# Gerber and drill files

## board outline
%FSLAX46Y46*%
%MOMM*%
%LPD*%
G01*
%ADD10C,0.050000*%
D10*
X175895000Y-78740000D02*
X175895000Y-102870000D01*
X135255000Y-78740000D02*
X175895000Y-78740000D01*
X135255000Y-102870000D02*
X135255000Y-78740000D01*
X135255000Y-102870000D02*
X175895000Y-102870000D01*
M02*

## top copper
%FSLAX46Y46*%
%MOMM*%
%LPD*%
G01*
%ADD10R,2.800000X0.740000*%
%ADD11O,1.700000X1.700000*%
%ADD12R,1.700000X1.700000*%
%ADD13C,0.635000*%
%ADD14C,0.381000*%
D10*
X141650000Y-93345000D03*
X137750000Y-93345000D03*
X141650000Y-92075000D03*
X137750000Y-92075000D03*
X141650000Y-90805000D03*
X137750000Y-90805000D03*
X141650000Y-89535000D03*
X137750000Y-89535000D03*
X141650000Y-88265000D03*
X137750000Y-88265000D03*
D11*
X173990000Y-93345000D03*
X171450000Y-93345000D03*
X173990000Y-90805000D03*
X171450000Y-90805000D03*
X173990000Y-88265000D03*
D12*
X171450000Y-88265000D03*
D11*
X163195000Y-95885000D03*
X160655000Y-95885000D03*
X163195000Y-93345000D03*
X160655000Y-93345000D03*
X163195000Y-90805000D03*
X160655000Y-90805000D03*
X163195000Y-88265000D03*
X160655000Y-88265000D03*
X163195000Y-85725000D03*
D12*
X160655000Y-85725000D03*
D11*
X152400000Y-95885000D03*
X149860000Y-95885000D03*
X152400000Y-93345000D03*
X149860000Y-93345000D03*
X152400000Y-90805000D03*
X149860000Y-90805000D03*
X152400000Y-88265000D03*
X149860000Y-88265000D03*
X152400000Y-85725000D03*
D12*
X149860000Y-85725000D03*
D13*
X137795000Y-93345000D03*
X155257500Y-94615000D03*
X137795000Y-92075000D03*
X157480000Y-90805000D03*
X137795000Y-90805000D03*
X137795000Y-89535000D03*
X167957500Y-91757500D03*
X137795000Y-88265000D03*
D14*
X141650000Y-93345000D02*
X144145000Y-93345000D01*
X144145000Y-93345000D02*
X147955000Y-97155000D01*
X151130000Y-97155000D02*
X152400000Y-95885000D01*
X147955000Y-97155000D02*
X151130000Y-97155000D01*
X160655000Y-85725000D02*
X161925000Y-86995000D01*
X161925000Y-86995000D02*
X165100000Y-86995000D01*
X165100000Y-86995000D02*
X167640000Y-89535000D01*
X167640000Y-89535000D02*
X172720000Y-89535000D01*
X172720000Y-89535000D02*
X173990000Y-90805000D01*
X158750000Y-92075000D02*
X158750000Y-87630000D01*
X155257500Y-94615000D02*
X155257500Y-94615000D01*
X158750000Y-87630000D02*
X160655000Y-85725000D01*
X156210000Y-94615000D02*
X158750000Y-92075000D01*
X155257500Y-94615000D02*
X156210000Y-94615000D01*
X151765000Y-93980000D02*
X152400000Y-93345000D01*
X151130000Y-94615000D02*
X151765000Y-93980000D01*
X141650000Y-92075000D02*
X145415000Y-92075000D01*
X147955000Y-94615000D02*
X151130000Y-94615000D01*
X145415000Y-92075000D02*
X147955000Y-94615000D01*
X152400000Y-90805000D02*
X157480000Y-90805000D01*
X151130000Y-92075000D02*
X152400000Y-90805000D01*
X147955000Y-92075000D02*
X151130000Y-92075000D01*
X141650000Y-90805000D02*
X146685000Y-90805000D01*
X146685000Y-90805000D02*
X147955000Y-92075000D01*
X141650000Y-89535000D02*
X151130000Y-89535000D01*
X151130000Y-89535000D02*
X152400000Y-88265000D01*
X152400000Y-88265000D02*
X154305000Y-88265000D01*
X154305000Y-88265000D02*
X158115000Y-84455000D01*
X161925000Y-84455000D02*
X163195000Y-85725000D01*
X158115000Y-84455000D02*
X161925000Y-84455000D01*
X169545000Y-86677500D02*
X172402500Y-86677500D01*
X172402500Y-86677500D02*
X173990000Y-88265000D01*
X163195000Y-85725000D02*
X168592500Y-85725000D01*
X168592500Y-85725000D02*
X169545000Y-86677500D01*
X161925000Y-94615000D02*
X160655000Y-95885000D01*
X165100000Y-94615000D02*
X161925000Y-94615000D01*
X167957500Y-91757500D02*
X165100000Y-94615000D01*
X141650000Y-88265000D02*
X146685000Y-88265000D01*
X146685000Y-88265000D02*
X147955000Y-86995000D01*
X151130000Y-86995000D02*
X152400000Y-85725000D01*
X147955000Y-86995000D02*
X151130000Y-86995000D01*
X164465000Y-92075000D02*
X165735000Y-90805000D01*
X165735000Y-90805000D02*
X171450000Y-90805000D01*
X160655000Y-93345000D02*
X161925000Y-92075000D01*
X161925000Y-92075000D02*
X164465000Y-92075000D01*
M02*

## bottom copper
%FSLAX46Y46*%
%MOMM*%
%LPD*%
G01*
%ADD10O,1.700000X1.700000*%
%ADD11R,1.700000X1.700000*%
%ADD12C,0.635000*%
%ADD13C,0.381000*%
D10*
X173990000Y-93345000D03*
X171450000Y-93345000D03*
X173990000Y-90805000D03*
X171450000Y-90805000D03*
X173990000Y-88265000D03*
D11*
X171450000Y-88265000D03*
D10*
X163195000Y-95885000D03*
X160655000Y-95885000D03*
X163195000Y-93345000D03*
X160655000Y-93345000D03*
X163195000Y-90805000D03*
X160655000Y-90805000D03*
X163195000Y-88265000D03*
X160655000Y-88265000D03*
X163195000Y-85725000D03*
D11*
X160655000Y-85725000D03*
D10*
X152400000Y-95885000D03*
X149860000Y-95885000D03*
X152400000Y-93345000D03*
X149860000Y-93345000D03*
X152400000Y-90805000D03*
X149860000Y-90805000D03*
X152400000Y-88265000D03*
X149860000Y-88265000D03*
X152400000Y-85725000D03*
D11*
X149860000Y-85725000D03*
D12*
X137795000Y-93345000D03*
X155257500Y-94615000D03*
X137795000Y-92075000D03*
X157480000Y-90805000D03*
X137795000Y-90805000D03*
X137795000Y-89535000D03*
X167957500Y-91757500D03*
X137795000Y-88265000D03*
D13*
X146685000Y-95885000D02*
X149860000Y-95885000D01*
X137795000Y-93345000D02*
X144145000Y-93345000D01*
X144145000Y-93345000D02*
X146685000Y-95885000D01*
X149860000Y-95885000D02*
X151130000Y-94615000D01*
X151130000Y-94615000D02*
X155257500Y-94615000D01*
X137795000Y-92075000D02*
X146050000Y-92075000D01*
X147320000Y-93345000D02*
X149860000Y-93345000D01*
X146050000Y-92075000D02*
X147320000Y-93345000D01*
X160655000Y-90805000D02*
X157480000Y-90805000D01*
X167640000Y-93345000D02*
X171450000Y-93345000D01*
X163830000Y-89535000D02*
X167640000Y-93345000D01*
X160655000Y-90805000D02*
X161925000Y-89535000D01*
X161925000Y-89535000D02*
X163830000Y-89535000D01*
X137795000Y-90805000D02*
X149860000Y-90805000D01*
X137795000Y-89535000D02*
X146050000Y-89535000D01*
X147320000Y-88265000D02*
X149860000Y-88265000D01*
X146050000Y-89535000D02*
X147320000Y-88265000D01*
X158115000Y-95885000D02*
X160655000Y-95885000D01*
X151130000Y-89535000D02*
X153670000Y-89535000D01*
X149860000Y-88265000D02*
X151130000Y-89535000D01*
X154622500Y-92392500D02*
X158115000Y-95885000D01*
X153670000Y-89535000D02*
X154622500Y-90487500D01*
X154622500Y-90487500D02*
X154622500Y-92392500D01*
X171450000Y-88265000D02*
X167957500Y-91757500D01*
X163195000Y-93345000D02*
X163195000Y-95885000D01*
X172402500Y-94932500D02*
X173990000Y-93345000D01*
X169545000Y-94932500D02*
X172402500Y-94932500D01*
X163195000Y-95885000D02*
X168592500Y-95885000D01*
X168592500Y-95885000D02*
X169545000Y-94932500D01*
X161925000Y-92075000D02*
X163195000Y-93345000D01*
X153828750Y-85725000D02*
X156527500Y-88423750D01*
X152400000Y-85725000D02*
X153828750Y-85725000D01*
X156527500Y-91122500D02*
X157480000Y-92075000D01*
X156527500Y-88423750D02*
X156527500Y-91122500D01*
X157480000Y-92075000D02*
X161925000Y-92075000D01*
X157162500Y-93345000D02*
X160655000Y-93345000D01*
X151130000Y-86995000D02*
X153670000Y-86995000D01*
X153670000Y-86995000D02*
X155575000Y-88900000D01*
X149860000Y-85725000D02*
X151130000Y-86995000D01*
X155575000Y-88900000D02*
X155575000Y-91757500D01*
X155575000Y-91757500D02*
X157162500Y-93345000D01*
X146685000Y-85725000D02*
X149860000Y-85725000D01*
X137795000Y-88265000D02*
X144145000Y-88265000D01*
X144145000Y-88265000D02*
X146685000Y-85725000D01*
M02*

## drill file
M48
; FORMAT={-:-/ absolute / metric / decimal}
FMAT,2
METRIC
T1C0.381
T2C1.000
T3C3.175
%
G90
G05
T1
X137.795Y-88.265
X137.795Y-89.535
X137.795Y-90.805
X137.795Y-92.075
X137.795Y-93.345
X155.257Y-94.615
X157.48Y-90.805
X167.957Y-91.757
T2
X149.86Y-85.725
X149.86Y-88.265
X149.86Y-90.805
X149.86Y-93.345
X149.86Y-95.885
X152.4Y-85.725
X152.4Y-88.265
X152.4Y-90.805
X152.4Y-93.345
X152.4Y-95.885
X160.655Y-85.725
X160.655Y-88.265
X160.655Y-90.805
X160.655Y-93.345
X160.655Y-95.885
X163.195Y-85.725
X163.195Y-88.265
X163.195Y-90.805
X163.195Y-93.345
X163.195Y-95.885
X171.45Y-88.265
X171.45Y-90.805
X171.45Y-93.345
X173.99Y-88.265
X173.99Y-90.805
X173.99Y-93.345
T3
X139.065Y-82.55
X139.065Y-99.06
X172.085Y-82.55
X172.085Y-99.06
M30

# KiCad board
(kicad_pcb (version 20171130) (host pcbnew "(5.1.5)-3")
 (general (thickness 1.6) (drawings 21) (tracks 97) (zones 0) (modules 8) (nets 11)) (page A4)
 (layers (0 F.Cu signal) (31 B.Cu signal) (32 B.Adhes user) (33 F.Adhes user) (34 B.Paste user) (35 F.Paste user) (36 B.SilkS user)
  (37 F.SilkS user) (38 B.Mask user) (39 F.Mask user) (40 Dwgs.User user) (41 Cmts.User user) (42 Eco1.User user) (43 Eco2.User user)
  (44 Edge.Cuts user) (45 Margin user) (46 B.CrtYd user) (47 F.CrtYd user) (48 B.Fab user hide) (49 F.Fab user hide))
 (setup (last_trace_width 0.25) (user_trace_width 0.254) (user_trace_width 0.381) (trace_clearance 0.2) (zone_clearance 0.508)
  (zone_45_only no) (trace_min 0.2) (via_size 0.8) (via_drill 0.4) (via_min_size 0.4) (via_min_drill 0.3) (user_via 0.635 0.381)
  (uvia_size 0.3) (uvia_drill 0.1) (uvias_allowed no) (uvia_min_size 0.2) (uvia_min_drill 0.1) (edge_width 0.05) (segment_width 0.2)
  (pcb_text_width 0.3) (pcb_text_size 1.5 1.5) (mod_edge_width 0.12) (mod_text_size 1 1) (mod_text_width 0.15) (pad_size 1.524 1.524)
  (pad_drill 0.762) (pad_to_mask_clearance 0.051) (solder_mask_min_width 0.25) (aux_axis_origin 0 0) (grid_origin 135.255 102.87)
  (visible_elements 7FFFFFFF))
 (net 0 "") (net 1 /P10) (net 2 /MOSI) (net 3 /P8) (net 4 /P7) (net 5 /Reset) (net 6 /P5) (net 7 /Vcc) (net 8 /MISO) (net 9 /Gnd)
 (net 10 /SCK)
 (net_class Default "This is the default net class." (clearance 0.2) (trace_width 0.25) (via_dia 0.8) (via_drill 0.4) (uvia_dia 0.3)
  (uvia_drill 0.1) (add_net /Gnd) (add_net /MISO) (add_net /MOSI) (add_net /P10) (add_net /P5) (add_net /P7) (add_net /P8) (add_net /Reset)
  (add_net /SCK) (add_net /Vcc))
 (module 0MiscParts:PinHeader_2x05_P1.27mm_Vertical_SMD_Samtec (layer F.Cu) (at 139.7 90.805)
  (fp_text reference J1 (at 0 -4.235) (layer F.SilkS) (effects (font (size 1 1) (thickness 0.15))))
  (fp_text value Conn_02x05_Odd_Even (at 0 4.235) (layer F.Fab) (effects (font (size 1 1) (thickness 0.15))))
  (pad 10 smd rect (at 1.95 2.54) (size 2.8 0.74) (layers F.Cu F.Paste F.Mask) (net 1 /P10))
  (pad 9 smd rect (at -1.95 2.54) (size 2.8 0.74) (layers F.Cu F.Paste F.Mask) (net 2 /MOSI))
  (pad 8 smd rect (at 1.95 1.27) (size 2.8 0.74) (layers F.Cu F.Paste F.Mask) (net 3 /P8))
  (pad 7 smd rect (at -1.95 1.27) (size 2.8 0.74) (layers F.Cu F.Paste F.Mask) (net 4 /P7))
  (pad 6 smd rect (at 1.95 0) (size 2.8 0.74) (layers F.Cu F.Paste F.Mask) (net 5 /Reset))
  (pad 5 smd rect (at -1.95 0) (size 2.8 0.74) (layers F.Cu F.Paste F.Mask) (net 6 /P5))
  (pad 4 smd rect (at 1.95 -1.27) (size 2.8 0.74) (layers F.Cu F.Paste F.Mask) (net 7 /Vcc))
  (pad 3 smd rect (at -1.95 -1.27) (size 2.8 0.74) (layers F.Cu F.Paste F.Mask) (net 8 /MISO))
  (pad 2 smd rect (at 1.95 -2.54) (size 2.8 0.74) (layers F.Cu F.Paste F.Mask) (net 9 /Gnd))
  (pad 1 smd rect (at -1.95 -2.54) (size 2.8 0.74) (layers F.Cu F.Paste F.Mask) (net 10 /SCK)))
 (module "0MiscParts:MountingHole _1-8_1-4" (layer F.Cu) (at 172.085 82.55)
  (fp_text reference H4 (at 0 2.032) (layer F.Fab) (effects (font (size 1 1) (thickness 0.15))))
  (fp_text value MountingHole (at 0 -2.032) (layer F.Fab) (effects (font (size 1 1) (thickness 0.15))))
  (pad "" np_thru_hole circle (at 0 0) (size 3.175 3.175) (drill 3.175) (layers *.Cu *.Mask)))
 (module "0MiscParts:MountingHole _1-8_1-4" (layer F.Cu) (at 172.085 99.06)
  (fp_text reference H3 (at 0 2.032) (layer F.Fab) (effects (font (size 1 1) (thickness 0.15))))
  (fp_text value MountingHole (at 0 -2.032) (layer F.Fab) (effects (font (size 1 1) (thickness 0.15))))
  (pad "" np_thru_hole circle (at 0 0) (size 3.175 3.175) (drill 3.175) (layers *.Cu *.Mask)))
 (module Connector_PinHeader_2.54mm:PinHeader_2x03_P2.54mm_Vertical (layer F.Cu) (at 171.45 88.265)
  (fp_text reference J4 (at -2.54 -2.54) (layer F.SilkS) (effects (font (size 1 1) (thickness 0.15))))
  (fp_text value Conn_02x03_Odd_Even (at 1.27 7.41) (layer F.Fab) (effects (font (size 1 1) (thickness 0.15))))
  (pad 6 thru_hole oval (at 2.54 5.08) (size 1.7 1.7) (drill 1) (layers *.Cu *.Mask) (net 9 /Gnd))
  (pad 5 thru_hole oval (at 0 5.08) (size 1.7 1.7) (drill 1) (layers *.Cu *.Mask) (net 5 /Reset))
  (pad 4 thru_hole oval (at 2.54 2.54) (size 1.7 1.7) (drill 1) (layers *.Cu *.Mask) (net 2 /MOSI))
  (pad 3 thru_hole oval (at 0 2.54) (size 1.7 1.7) (drill 1) (layers *.Cu *.Mask) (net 10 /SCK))
  (pad 2 thru_hole oval (at 2.54 0) (size 1.7 1.7) (drill 1) (layers *.Cu *.Mask) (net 7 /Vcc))
  (pad 1 thru_hole rect (at 0 0) (size 1.7 1.7) (drill 1) (layers *.Cu *.Mask) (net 8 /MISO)))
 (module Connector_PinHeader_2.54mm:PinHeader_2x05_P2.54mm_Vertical (layer F.Cu) (at 160.655 85.725)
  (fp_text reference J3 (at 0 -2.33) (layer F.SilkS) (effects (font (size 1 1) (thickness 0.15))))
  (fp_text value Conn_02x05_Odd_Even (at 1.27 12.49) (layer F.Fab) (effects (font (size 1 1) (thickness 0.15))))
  (pad 10 thru_hole oval (at 2.54 10.16) (size 1.7 1.7) (drill 1) (layers *.Cu *.Mask) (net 9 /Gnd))
  (pad 9 thru_hole oval (at 0 10.16) (size 1.7 1.7) (drill 1) (layers *.Cu *.Mask) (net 8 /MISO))
  (pad 8 thru_hole oval (at 2.54 7.62) (size 1.7 1.7) (drill 1) (layers *.Cu *.Mask) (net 9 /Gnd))
  (pad 7 thru_hole oval (at 0 7.62) (size 1.7 1.7) (drill 1) (layers *.Cu *.Mask) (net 10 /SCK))
  (pad 6 thru_hole oval (at 2.54 5.08) (size 1.7 1.7) (drill 1) (layers *.Cu *.Mask))
  (pad 5 thru_hole oval (at 0 5.08) (size 1.7 1.7) (drill 1) (layers *.Cu *.Mask) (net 5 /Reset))
  (pad 4 thru_hole oval (at 2.54 2.54) (size 1.7 1.7) (drill 1) (layers *.Cu *.Mask))
  (pad 3 thru_hole oval (at 0 2.54) (size 1.7 1.7) (drill 1) (layers *.Cu *.Mask))
  (pad 2 thru_hole oval (at 2.54 0) (size 1.7 1.7) (drill 1) (layers *.Cu *.Mask) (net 7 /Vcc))
  (pad 1 thru_hole rect (at 0 0) (size 1.7 1.7) (drill 1) (layers *.Cu *.Mask) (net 2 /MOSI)))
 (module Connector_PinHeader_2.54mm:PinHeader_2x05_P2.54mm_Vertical (layer F.Cu) (at 149.86 85.725)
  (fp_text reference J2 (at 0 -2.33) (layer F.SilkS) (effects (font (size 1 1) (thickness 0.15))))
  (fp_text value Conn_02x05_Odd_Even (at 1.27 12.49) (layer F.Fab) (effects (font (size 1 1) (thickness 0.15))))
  (pad 10 thru_hole oval (at 2.54 10.16) (size 1.7 1.7) (drill 1) (layers *.Cu *.Mask) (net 1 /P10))
  (pad 9 thru_hole oval (at 0 10.16) (size 1.7 1.7) (drill 1) (layers *.Cu *.Mask) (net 2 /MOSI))
  (pad 8 thru_hole oval (at 2.54 7.62) (size 1.7 1.7) (drill 1) (layers *.Cu *.Mask) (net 3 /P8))
  (pad 7 thru_hole oval (at 0 7.62) (size 1.7 1.7) (drill 1) (layers *.Cu *.Mask) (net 4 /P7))
  (pad 6 thru_hole oval (at 2.54 5.08) (size 1.7 1.7) (drill 1) (layers *.Cu *.Mask) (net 5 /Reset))
  (pad 5 thru_hole oval (at 0 5.08) (size 1.7 1.7) (drill 1) (layers *.Cu *.Mask) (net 6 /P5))
  (pad 4 thru_hole oval (at 2.54 2.54) (size 1.7 1.7) (drill 1) (layers *.Cu *.Mask) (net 7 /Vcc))
  (pad 3 thru_hole oval (at 0 2.54) (size 1.7 1.7) (drill 1) (layers *.Cu *.Mask) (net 8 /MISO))
  (pad 2 thru_hole oval (at 2.54 0) (size 1.7 1.7) (drill 1) (layers *.Cu *.Mask) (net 9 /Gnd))
  (pad 1 thru_hole rect (at 0 0) (size 1.7 1.7) (drill 1) (layers *.Cu *.Mask) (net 10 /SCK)))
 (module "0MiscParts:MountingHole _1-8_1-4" (layer F.Cu) (at 139.065 82.55)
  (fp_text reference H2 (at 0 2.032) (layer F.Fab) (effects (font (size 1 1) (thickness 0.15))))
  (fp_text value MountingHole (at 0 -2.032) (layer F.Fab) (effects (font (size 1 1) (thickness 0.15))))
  (pad "" np_thru_hole circle (at 0 0) (size 3.175 3.175) (drill 3.175) (layers *.Cu *.Mask)))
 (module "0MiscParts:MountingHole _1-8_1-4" (layer F.Cu) (at 139.065 99.06)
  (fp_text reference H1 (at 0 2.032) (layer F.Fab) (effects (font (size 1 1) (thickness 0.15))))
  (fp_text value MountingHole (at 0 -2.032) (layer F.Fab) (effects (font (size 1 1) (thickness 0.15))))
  (pad "" np_thru_hole circle (at 0 0) (size 3.175 3.175) (drill 3.175) (layers *.Cu *.Mask)))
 (gr_line (start 175.895 78.74) (end 175.895 102.87) (layer Edge.Cuts) (width 0.05))
 (gr_line (start 135.255 78.74) (end 175.895 78.74) (layer Edge.Cuts) (width 0.05))
 (gr_line (start 135.255 102.87) (end 135.255 78.74) (layer Edge.Cuts) (width 0.05))
 (gr_line (start 135.255 102.87) (end 175.895 102.87) (layer Edge.Cuts) (width 0.05))
 (segment (start 141.65 93.345) (end 144.145 93.345) (width 0.381) (layer F.Cu) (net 1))
 (segment (start 144.145 93.345) (end 147.955 97.155) (width 0.381) (layer F.Cu) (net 1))
 (segment (start 151.13 97.155) (end 152.4 95.885) (width 0.381) (layer F.Cu) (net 1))
 (segment (start 147.955 97.155) (end 151.13 97.155) (width 0.381) (layer F.Cu) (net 1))
 (via (at 137.795 93.345) (size 0.635) (drill 0.381) (layers F.Cu B.Cu) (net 2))
 (segment (start 160.655 85.725) (end 161.925 86.995) (width 0.381) (layer F.Cu) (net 2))
 (segment (start 161.925 86.995) (end 165.1 86.995) (width 0.381) (layer F.Cu) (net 2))
 (segment (start 165.1 86.995) (end 167.64 89.535) (width 0.381) (layer F.Cu) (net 2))
 (segment (start 167.64 89.535) (end 172.72 89.535) (width 0.381) (layer F.Cu) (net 2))
 (segment (start 172.72 89.535) (end 173.99 90.805) (width 0.381) (layer F.Cu) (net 2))
 (segment (start 146.685 95.885) (end 149.86 95.885) (width 0.381) (layer B.Cu) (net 2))
 (segment (start 137.795 93.345) (end 144.145 93.345) (width 0.381) (layer B.Cu) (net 2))
 (segment (start 144.145 93.345) (end 146.685 95.885) (width 0.381) (layer B.Cu) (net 2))
 (segment (start 158.75 92.075) (end 158.75 87.63) (width 0.381) (layer F.Cu) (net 2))
 (segment (start 155.2575 94.615) (end 155.2575 94.615) (width 0.381) (layer F.Cu) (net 2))
 (segment (start 158.75 87.63) (end 160.655 85.725) (width 0.381) (layer F.Cu) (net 2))
 (segment (start 156.21 94.615) (end 158.75 92.075) (width 0.381) (layer F.Cu) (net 2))
 (segment (start 155.2575 94.615) (end 156.21 94.615) (width 0.381) (layer F.Cu) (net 2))
 (via (at 155.2575 94.615) (size 0.635) (drill 0.381) (layers F.Cu B.Cu) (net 2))
 (segment (start 149.86 95.885) (end 151.13 94.615) (width 0.381) (layer B.Cu) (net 2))
 (segment (start 151.13 94.615) (end 155.2575 94.615) (width 0.381) (layer B.Cu) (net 2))
 (segment (start 151.765 93.98) (end 152.4 93.345) (width 0.381) (layer F.Cu) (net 3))
 (segment (start 151.13 94.615) (end 151.765 93.98) (width 0.381) (layer F.Cu) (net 3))
 (segment (start 141.65 92.075) (end 145.415 92.075) (width 0.381) (layer F.Cu) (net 3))
 (segment (start 147.955 94.615) (end 151.13 94.615) (width 0.381) (layer F.Cu) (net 3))
 (segment (start 145.415 92.075) (end 147.955 94.615) (width 0.381) (layer F.Cu) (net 3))
 (via (at 137.795 92.075) (size 0.635) (drill 0.381) (layers F.Cu B.Cu) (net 4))
 (segment (start 137.795 92.075) (end 146.05 92.075) (width 0.381) (layer B.Cu) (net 4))
 (segment (start 147.32 93.345) (end 149.86 93.345) (width 0.381) (layer B.Cu) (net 4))
 (segment (start 146.05 92.075) (end 147.32 93.345) (width 0.381) (layer B.Cu) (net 4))
 (via (at 157.48 90.805) (size 0.635) (drill 0.381) (layers F.Cu B.Cu) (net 5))
 (segment (start 160.655 90.805) (end 157.48 90.805) (width 0.381) (layer B.Cu) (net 5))
 (segment (start 152.4 90.805) (end 157.48 90.805) (width 0.381) (layer F.Cu) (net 5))
 (segment (start 151.13 92.075) (end 152.4 90.805) (width 0.381) (layer F.Cu) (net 5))
 (segment (start 147.955 92.075) (end 151.13 92.075) (width 0.381) (layer F.Cu) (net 5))
 (segment (start 141.65 90.805) (end 146.685 90.805) (width 0.381) (layer F.Cu) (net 5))
 (segment (start 146.685 90.805) (end 147.955 92.075) (width 0.381) (layer F.Cu) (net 5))
 (segment (start 167.64 93.345) (end 171.45 93.345) (width 0.381) (layer B.Cu) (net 5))
 (segment (start 163.83 89.535) (end 167.64 93.345) (width 0.381) (layer B.Cu) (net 5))
 (segment (start 160.655 90.805) (end 161.925 89.535) (width 0.381) (layer B.Cu) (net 5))
 (segment (start 161.925 89.535) (end 163.83 89.535) (width 0.381) (layer B.Cu) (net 5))
 (via (at 137.795 90.805) (size 0.635) (drill 0.381) (layers F.Cu B.Cu) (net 6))
 (segment (start 137.795 90.805) (end 149.86 90.805) (width 0.381) (layer B.Cu) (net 6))
 (segment (start 141.65 89.535) (end 151.13 89.535) (width 0.381) (layer F.Cu) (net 7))
 (segment (start 151.13 89.535) (end 152.4 88.265) (width 0.381) (layer F.Cu) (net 7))
 (segment (start 152.4 88.265) (end 154.305 88.265) (width 0.381) (layer F.Cu) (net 7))
 (segment (start 154.305 88.265) (end 158.115 84.455) (width 0.381) (layer F.Cu) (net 7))
 (segment (start 161.925 84.455) (end 163.195 85.725) (width 0.381) (layer F.Cu) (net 7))
 (segment (start 158.115 84.455) (end 161.925 84.455) (width 0.381) (layer F.Cu) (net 7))
 (segment (start 169.545 86.6775) (end 172.4025 86.6775) (width 0.381) (layer F.Cu) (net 7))
 (segment (start 172.4025 86.6775) (end 173.99 88.265) (width 0.381) (layer F.Cu) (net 7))
 (segment (start 163.195 85.725) (end 168.5925 85.725) (width 0.381) (layer F.Cu) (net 7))
 (segment (start 168.5925 85.725) (end 169.545 86.6775) (width 0.381) (layer F.Cu) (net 7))
 (via (at 137.795 89.535) (size 0.635) (drill 0.381) (layers F.Cu B.Cu) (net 8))
 (segment (start 137.795 89.535) (end 146.05 89.535) (width 0.381) (layer B.Cu) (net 8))
 (segment (start 147.32 88.265) (end 149.86 88.265) (width 0.381) (layer B.Cu) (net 8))
 (segment (start 146.05 89.535) (end 147.32 88.265) (width 0.381) (layer B.Cu) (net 8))
 (segment (start 158.115 95.885) (end 160.655 95.885) (width 0.381) (layer B.Cu) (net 8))
 (segment (start 151.13 89.535) (end 153.67 89.535) (width 0.381) (layer B.Cu) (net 8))
 (segment (start 149.86 88.265) (end 151.13 89.535) (width 0.381) (layer B.Cu) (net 8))
 (segment (start 154.6225 92.3925) (end 158.115 95.885) (width 0.381) (layer B.Cu) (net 8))
 (segment (start 153.67 89.535) (end 154.6225 90.4875) (width 0.381) (layer B.Cu) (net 8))
 (segment (start 154.6225 90.4875) (end 154.6225 92.3925) (width 0.381) (layer B.Cu) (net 8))
 (segment (start 161.925 94.615) (end 160.655 95.885) (width 0.381) (layer F.Cu) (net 8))
 (segment (start 171.45 88.265) (end 167.9575 91.7575) (width 0.381) (layer B.Cu) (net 8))
 (segment (start 165.1 94.615) (end 161.925 94.615) (width 0.381) (layer F.Cu) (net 8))
 (via (at 167.9575 91.7575) (size 0.635) (drill 0.381) (layers F.Cu B.Cu) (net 8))
 (segment (start 167.9575 91.7575) (end 165.1 94.615) (width 0.381) (layer F.Cu) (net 8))
 (segment (start 141.65 88.265) (end 146.685 88.265) (width 0.381) (layer F.Cu) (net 9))
 (segment (start 146.685 88.265) (end 147.955 86.995) (width 0.381) (layer F.Cu) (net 9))
 (segment (start 151.13 86.995) (end 152.4 85.725) (width 0.381) (layer F.Cu) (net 9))
 (segment (start 147.955 86.995) (end 151.13 86.995) (width 0.381) (layer F.Cu) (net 9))
 (segment (start 163.195 93.345) (end 163.195 95.885) (width 0.381) (layer B.Cu) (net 9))
 (segment (start 172.4025 94.9325) (end 173.99 93.345) (width 0.381) (layer B.Cu) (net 9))
 (segment (start 169.545 94.9325) (end 172.4025 94.9325) (width 0.381) (layer B.Cu) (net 9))
 (segment (start 163.195 95.885) (end 168.5925 95.885) (width 0.381) (layer B.Cu) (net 9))
 (segment (start 168.5925 95.885) (end 169.545 94.9325) (width 0.381) (layer B.Cu) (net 9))
 (segment (start 161.925 92.075) (end 163.195 93.345) (width 0.381) (layer B.Cu) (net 9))
 (segment (start 153.82875 85.725) (end 156.5275 88.42375) (width 0.381) (layer B.Cu) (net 9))
 (segment (start 152.4 85.725) (end 153.82875 85.725) (width 0.381) (layer B.Cu) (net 9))
 (segment (start 156.5275 91.1225) (end 157.48 92.075) (width 0.381) (layer B.Cu) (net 9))
 (segment (start 156.5275 88.42375) (end 156.5275 91.1225) (width 0.381) (layer B.Cu) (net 9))
 (segment (start 157.48 92.075) (end 161.925 92.075) (width 0.381) (layer B.Cu) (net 9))
 (via (at 137.795 88.265) (size 0.635) (drill 0.381) (layers F.Cu B.Cu) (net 10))
 (segment (start 164.465 92.075) (end 165.735 90.805) (width 0.381) (layer F.Cu) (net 10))
 (segment (start 165.735 90.805) (end 171.45 90.805) (width 0.381) (layer F.Cu) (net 10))
 (segment (start 160.655 93.345) (end 161.925 92.075) (width 0.381) (layer F.Cu) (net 10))
 (segment (start 161.925 92.075) (end 164.465 92.075) (width 0.381) (layer F.Cu) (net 10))
 (segment (start 157.1625 93.345) (end 160.655 93.345) (width 0.381) (layer B.Cu) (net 10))
 (segment (start 151.13 86.995) (end 153.67 86.995) (width 0.381) (layer B.Cu) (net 10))
 (segment (start 153.67 86.995) (end 155.575 88.9) (width 0.381) (layer B.Cu) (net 10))
 (segment (start 149.86 85.725) (end 151.13 86.995) (width 0.381) (layer B.Cu) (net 10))
 (segment (start 155.575 88.9) (end 155.575 91.7575) (width 0.381) (layer B.Cu) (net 10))
 (segment (start 155.575 91.7575) (end 157.1625 93.345) (width 0.381) (layer B.Cu) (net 10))
 (segment (start 146.685 85.725) (end 149.86 85.725) (width 0.381) (layer B.Cu) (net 10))
 (segment (start 137.795 88.265) (end 144.145 88.265) (width 0.381) (layer B.Cu) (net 10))
 (segment (start 144.145 88.265) (end 146.685 85.725) (width 0.381) (layer B.Cu) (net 10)))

